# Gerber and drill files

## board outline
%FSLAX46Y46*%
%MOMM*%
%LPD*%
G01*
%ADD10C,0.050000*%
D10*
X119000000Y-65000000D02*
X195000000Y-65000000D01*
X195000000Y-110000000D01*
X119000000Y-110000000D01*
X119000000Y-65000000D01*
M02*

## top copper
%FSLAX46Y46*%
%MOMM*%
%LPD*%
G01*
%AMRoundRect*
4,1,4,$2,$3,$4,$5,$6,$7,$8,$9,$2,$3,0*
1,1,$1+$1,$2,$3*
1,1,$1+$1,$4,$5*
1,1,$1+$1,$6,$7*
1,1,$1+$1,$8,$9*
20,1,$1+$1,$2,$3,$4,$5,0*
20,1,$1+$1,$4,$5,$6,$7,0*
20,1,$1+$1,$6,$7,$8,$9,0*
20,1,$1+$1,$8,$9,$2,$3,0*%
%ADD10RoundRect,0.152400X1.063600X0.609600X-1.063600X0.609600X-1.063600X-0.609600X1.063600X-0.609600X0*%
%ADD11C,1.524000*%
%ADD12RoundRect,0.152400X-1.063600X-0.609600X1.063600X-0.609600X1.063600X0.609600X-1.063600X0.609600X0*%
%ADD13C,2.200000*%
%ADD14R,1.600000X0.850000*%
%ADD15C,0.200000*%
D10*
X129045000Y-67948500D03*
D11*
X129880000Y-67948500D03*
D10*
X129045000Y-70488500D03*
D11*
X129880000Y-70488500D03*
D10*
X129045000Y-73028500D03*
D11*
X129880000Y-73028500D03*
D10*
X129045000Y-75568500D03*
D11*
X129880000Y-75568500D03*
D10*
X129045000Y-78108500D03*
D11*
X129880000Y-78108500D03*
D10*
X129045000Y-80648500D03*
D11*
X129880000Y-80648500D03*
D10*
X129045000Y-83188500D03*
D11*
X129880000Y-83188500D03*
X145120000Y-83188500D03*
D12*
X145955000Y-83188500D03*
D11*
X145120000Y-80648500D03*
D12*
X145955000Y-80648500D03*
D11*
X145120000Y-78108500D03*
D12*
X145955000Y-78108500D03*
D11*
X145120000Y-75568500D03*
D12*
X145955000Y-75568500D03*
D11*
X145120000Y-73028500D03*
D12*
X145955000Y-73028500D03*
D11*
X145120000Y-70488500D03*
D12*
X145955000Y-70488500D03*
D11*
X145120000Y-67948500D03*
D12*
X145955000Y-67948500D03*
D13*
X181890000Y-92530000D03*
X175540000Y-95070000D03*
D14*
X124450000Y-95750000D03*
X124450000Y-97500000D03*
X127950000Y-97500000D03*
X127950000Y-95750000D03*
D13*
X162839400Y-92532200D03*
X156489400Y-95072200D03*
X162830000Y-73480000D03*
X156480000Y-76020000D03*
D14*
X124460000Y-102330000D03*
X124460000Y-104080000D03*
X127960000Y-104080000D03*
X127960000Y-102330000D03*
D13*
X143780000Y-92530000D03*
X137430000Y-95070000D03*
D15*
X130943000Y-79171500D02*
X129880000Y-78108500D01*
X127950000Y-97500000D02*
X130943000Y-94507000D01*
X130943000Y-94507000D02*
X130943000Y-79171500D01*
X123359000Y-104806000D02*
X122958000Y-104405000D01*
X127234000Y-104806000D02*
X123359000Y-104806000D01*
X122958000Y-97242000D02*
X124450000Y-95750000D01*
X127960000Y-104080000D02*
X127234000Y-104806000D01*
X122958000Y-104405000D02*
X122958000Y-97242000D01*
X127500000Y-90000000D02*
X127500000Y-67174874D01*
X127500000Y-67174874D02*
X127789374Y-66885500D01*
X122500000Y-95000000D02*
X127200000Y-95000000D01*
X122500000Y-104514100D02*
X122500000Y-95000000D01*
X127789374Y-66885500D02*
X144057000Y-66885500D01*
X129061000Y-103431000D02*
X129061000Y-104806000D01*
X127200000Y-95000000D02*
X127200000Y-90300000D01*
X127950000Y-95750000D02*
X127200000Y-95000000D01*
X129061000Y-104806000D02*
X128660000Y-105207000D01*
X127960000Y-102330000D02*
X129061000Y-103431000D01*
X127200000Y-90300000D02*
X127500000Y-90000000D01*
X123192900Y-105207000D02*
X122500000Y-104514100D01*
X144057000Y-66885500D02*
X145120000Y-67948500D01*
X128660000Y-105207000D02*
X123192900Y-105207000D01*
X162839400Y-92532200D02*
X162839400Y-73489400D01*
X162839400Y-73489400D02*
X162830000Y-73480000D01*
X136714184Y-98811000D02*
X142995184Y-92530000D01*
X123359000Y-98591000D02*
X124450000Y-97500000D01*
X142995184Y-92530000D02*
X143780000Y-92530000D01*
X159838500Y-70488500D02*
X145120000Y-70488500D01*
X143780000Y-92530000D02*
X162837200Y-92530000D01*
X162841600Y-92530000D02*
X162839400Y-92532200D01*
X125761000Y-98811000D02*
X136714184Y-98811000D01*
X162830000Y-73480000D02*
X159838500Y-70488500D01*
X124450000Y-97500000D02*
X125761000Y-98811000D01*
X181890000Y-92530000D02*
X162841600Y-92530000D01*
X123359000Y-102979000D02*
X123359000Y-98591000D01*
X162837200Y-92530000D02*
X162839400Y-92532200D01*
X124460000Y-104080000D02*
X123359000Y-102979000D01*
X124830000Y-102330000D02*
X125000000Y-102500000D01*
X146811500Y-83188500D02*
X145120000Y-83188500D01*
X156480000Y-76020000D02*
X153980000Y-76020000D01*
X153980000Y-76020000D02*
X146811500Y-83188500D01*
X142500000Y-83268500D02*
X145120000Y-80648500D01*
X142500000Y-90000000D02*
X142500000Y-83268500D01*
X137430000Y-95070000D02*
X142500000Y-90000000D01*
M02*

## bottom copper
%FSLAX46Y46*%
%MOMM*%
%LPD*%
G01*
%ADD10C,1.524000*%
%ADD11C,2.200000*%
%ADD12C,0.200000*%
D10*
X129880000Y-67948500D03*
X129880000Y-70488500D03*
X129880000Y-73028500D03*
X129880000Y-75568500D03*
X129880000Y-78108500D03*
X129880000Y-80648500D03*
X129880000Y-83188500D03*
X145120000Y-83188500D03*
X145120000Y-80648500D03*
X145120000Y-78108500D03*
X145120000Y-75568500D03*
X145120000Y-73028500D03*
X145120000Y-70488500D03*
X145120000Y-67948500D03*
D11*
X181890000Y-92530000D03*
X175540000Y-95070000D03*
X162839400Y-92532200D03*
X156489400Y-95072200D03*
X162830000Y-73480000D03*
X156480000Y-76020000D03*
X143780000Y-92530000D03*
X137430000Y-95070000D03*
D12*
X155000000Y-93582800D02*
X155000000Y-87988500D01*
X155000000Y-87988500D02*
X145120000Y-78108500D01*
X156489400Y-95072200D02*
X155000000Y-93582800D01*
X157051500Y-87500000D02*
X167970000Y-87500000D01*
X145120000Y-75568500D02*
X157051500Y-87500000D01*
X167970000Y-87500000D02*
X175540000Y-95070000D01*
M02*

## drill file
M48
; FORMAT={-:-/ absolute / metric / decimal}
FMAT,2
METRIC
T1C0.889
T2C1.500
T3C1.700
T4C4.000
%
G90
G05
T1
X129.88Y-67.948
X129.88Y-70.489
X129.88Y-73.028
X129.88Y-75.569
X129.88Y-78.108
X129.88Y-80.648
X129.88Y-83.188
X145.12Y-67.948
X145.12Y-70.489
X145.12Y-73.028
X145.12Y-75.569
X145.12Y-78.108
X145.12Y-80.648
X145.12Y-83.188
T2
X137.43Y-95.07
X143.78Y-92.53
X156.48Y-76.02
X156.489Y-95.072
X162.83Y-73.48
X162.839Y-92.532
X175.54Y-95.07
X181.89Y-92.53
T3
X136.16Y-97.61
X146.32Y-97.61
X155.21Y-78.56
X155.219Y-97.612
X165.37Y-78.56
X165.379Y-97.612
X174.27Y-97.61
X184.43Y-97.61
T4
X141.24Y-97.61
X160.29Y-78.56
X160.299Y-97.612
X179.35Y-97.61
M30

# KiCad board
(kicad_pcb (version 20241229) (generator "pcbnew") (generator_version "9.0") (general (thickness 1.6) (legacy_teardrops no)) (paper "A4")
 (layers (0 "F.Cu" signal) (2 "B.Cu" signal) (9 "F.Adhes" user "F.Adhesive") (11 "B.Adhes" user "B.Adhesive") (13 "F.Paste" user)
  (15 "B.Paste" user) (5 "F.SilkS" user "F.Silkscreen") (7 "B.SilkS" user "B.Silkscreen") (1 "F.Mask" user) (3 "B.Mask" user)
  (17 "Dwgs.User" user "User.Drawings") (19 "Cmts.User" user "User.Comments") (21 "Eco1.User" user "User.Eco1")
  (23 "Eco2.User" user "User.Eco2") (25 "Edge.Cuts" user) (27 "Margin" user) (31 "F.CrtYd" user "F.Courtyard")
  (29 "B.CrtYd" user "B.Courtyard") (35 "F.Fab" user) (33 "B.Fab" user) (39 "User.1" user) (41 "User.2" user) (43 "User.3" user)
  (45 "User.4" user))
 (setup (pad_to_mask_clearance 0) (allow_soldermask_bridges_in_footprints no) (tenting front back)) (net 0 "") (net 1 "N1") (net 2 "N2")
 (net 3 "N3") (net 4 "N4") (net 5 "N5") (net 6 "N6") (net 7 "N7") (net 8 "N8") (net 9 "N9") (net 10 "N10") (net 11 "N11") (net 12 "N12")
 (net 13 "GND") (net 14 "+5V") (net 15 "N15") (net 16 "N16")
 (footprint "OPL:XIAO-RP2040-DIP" (layer "F.Cu") (at 137.5 75.5685)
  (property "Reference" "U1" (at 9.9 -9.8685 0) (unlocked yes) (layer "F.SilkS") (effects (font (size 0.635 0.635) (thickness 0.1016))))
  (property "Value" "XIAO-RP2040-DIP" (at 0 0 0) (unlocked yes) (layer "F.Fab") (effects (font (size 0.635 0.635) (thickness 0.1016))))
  (pad "1" smd roundrect (at -8.455 -7.62 180) (size 2.432 1.524) (layers "F.Cu" "F.Mask") (roundrect_rratio 0.1) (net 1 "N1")
   (thermal_bridge_angle 45))
  (pad "1" thru_hole circle (at -7.62 -7.62 180) (size 1.524 1.524) (drill 0.889) (layers "*.Cu" "*.Mask") (remove_unused_layers no)
   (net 1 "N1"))
  (pad "2" smd roundrect (at -8.455 -5.08 180) (size 2.432 1.524) (layers "F.Cu" "F.Mask") (roundrect_rratio 0.1) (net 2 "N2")
   (thermal_bridge_angle 45))
  (pad "2" thru_hole circle (at -7.62 -5.08 180) (size 1.524 1.524) (drill 0.889) (layers "*.Cu" "*.Mask") (remove_unused_layers no)
   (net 2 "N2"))
  (pad "3" smd roundrect (at -8.455 -2.54 180) (size 2.432 1.524) (layers "F.Cu" "F.Mask") (roundrect_rratio 0.1) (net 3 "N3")
   (thermal_bridge_angle 45))
  (pad "3" thru_hole circle (at -7.62 -2.54 180) (size 1.524 1.524) (drill 0.889) (layers "*.Cu" "*.Mask") (remove_unused_layers no)
   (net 3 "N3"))
  (pad "4" smd roundrect (at -8.455 0 180) (size 2.432 1.524) (layers "F.Cu" "F.Mask") (roundrect_rratio 0.1) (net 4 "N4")
   (thermal_bridge_angle 45))
  (pad "4" thru_hole circle (at -7.62 0 180) (size 1.524 1.524) (drill 0.889) (layers "*.Cu" "*.Mask") (remove_unused_layers no)
   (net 4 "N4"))
  (pad "5" smd roundrect (at -8.455 2.54 180) (size 2.432 1.524) (layers "F.Cu" "F.Mask") (roundrect_rratio 0.1) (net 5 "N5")
   (thermal_bridge_angle 45))
  (pad "5" thru_hole circle (at -7.62 2.54 180) (size 1.524 1.524) (drill 0.889) (layers "*.Cu" "*.Mask") (remove_unused_layers no)
   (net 5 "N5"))
  (pad "6" smd roundrect (at -8.455 5.08 180) (size 2.432 1.524) (layers "F.Cu" "F.Mask") (roundrect_rratio 0.1) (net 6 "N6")
   (thermal_bridge_angle 45))
  (pad "6" thru_hole circle (at -7.62 5.08 180) (size 1.524 1.524) (drill 0.889) (layers "*.Cu" "*.Mask") (remove_unused_layers no)
   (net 6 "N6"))
  (pad "7" smd roundrect (at -8.455 7.62 180) (size 2.432 1.524) (layers "F.Cu" "F.Mask") (roundrect_rratio 0.1) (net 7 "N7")
   (thermal_bridge_angle 45))
  (pad "7" thru_hole circle (at -7.62 7.62 180) (size 1.524 1.524) (drill 0.889) (layers "*.Cu" "*.Mask") (remove_unused_layers no)
   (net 7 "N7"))
  (pad "8" thru_hole circle (at 7.62 7.62) (size 1.524 1.524) (drill 0.889) (layers "*.Cu" "*.Mask") (remove_unused_layers no) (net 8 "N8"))
  (pad "8" smd roundrect (at 8.455 7.62) (size 2.432 1.524) (layers "F.Cu" "F.Mask") (roundrect_rratio 0.1) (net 8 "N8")
   (thermal_bridge_angle 45))
  (pad "9" thru_hole circle (at 7.62 5.08) (size 1.524 1.524) (drill 0.889) (layers "*.Cu" "*.Mask") (remove_unused_layers no) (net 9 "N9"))
  (pad "9" smd roundrect (at 8.455 5.08) (size 2.432 1.524) (layers "F.Cu" "F.Mask") (roundrect_rratio 0.1) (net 9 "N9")
   (thermal_bridge_angle 45))
  (pad "10" thru_hole circle (at 7.62 2.54) (size 1.524 1.524) (drill 0.889) (layers "*.Cu" "*.Mask") (remove_unused_layers no)
   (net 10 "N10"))
  (pad "10" smd roundrect (at 8.455 2.54) (size 2.432 1.524) (layers "F.Cu" "F.Mask") (roundrect_rratio 0.1) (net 10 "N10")
   (thermal_bridge_angle 45))
  (pad "11" thru_hole circle (at 7.62 0) (size 1.524 1.524) (drill 0.889) (layers "*.Cu" "*.Mask") (remove_unused_layers no) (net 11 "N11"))
  (pad "11" smd roundrect (at 8.455 0) (size 2.432 1.524) (layers "F.Cu" "F.Mask") (roundrect_rratio 0.1) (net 11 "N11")
   (thermal_bridge_angle 45))
  (pad "12" thru_hole circle (at 7.62 -2.54) (size 1.524 1.524) (drill 0.889) (layers "*.Cu" "*.Mask") (remove_unused_layers no)
   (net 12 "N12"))
  (pad "12" smd roundrect (at 8.455 -2.54) (size 2.432 1.524) (layers "F.Cu" "F.Mask") (roundrect_rratio 0.1) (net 12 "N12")
   (thermal_bridge_angle 45))
  (pad "13" thru_hole circle (at 7.62 -5.08) (size 1.524 1.524) (drill 0.889) (layers "*.Cu" "*.Mask") (remove_unused_layers no)
   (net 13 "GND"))
  (pad "13" smd roundrect (at 8.455 -5.08) (size 2.432 1.524) (layers "F.Cu" "F.Mask") (roundrect_rratio 0.1) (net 13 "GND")
   (thermal_bridge_angle 45))
  (pad "14" thru_hole circle (at 7.62 -7.62) (size 1.524 1.524) (drill 0.889) (layers "*.Cu" "*.Mask") (remove_unused_layers no)
   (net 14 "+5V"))
  (pad "14" smd roundrect (at 8.455 -7.62) (size 2.432 1.524) (layers "F.Cu" "F.Mask") (roundrect_rratio 0.1) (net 14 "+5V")
   (thermal_bridge_angle 45)))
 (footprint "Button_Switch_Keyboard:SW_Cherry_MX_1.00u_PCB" (layer "F.Cu") (at 181.89 92.53)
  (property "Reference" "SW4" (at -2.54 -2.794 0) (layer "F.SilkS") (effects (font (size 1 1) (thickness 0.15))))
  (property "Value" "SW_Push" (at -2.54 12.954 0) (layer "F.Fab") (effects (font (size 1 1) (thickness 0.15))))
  (pad "" np_thru_hole circle (at -7.62 5.08) (size 1.7 1.7) (drill 1.7) (layers "*.Cu" "*.Mask"))
  (pad "" np_thru_hole circle (at -2.54 5.08) (size 4 4) (drill 4) (layers "*.Cu" "*.Mask"))
  (pad "" np_thru_hole circle (at 2.54 5.08) (size 1.7 1.7) (drill 1.7) (layers "*.Cu" "*.Mask"))
  (pad "1" thru_hole circle (at 0 0) (size 2.2 2.2) (drill 1.5) (layers "*.Cu" "*.Mask") (remove_unused_layers no) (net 13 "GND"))
  (pad "2" thru_hole circle (at -6.35 2.54) (size 2.2 2.2) (drill 1.5) (layers "*.Cu" "*.Mask") (remove_unused_layers no) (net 11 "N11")))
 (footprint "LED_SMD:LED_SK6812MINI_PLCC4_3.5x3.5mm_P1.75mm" (layer "F.Cu") (at 126.2 96.625)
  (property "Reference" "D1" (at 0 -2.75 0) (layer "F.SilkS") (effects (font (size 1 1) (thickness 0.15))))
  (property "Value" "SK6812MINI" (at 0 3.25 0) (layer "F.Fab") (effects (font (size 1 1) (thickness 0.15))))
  (pad "1" smd rect (at -1.75 -0.875) (size 1.6 0.85) (layers "F.Cu" "F.Mask" "F.Paste") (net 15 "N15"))
  (pad "2" smd rect (at -1.75 0.875) (size 1.6 0.85) (layers "F.Cu" "F.Mask" "F.Paste") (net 13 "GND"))
  (pad "3" smd rect (at 1.75 0.875) (size 1.6 0.85) (layers "F.Cu" "F.Mask" "F.Paste") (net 5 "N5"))
  (pad "4" smd rect (at 1.75 -0.875) (size 1.6 0.85) (layers "F.Cu" "F.Mask" "F.Paste") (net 14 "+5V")))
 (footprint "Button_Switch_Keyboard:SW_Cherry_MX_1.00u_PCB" (layer "F.Cu") (at 162.8394 92.5322)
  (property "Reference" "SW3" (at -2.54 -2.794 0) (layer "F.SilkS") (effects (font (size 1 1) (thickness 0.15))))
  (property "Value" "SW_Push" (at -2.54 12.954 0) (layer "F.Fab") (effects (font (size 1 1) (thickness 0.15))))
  (pad "" np_thru_hole circle (at -7.62 5.08) (size 1.7 1.7) (drill 1.7) (layers "*.Cu" "*.Mask"))
  (pad "" np_thru_hole circle (at -2.54 5.08) (size 4 4) (drill 4) (layers "*.Cu" "*.Mask"))
  (pad "" np_thru_hole circle (at 2.54 5.08) (size 1.7 1.7) (drill 1.7) (layers "*.Cu" "*.Mask"))
  (pad "1" thru_hole circle (at 0 0) (size 2.2 2.2) (drill 1.5) (layers "*.Cu" "*.Mask") (remove_unused_layers no) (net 13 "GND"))
  (pad "2" thru_hole circle (at -6.35 2.54) (size 2.2 2.2) (drill 1.5) (layers "*.Cu" "*.Mask") (remove_unused_layers no) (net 10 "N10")))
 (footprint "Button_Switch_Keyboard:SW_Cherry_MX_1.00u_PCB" (layer "F.Cu") (at 162.83 73.48)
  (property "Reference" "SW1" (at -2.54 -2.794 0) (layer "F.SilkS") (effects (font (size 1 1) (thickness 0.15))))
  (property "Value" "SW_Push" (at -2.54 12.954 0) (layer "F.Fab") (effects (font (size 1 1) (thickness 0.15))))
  (pad "" np_thru_hole circle (at -7.62 5.08) (size 1.7 1.7) (drill 1.7) (layers "*.Cu" "*.Mask"))
  (pad "" np_thru_hole circle (at -2.54 5.08) (size 4 4) (drill 4) (layers "*.Cu" "*.Mask"))
  (pad "" np_thru_hole circle (at 2.54 5.08) (size 1.7 1.7) (drill 1.7) (layers "*.Cu" "*.Mask"))
  (pad "1" thru_hole circle (at 0 0) (size 2.2 2.2) (drill 1.5) (layers "*.Cu" "*.Mask") (remove_unused_layers no) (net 13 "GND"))
  (pad "2" thru_hole circle (at -6.35 2.54) (size 2.2 2.2) (drill 1.5) (layers "*.Cu" "*.Mask") (remove_unused_layers no) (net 8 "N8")))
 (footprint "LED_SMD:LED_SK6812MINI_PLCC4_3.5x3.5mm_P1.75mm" (layer "F.Cu") (at 126.21 103.205)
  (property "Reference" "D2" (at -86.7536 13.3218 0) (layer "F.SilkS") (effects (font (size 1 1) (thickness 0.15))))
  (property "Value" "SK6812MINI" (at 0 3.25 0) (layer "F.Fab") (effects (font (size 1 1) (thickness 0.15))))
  (pad "1" smd rect (at -1.75 -0.875) (size 1.6 0.85) (layers "F.Cu" "F.Mask" "F.Paste") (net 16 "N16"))
  (pad "2" smd rect (at -1.75 0.875) (size 1.6 0.85) (layers "F.Cu" "F.Mask" "F.Paste") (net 13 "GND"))
  (pad "3" smd rect (at 1.75 0.875) (size 1.6 0.85) (layers "F.Cu" "F.Mask" "F.Paste") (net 15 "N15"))
  (pad "4" smd rect (at 1.75 -0.875) (size 1.6 0.85) (layers "F.Cu" "F.Mask" "F.Paste") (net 14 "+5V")))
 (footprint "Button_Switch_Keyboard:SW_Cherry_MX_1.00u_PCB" (layer "F.Cu") (at 143.78 92.53)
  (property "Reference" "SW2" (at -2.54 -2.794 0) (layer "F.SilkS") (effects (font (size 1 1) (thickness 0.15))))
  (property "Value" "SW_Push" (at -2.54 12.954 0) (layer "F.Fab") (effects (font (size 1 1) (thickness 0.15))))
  (pad "" np_thru_hole circle (at -7.62 5.08) (size 1.7 1.7) (drill 1.7) (layers "*.Cu" "*.Mask"))
  (pad "" np_thru_hole circle (at -2.54 5.08) (size 4 4) (drill 4) (layers "*.Cu" "*.Mask"))
  (pad "" np_thru_hole circle (at 2.54 5.08) (size 1.7 1.7) (drill 1.7) (layers "*.Cu" "*.Mask"))
  (pad "1" thru_hole circle (at 0 0) (size 2.2 2.2) (drill 1.5) (layers "*.Cu" "*.Mask") (remove_unused_layers no) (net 13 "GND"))
  (pad "2" thru_hole circle (at -6.35 2.54) (size 2.2 2.2) (drill 1.5) (layers "*.Cu" "*.Mask") (remove_unused_layers no) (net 9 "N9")))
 (gr_rect (start 119 65) (end 195 110) (stroke (width 0.05) (type default)) (fill no) (layer "Edge.Cuts"))
 (segment (start 130.943 79.1715) (end 129.88 78.1085) (width 0.2) (layer "F.Cu") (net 5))
 (segment (start 127.95 97.5) (end 130.943 94.507) (width 0.2) (layer "F.Cu") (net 5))
 (segment (start 130.943 94.507) (end 130.943 79.1715) (width 0.2) (layer "F.Cu") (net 5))
 (segment (start 123.359 104.806) (end 122.958 104.405) (width 0.2) (layer "F.Cu") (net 15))
 (segment (start 127.234 104.806) (end 123.359 104.806) (width 0.2) (layer "F.Cu") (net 15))
 (segment (start 122.958 97.242) (end 124.45 95.75) (width 0.2) (layer "F.Cu") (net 15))
 (segment (start 127.96 104.08) (end 127.234 104.806) (width 0.2) (layer "F.Cu") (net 15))
 (segment (start 122.958 104.405) (end 122.958 97.242) (width 0.2) (layer "F.Cu") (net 15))
 (segment (start 127.5 90) (end 127.5 67.174874) (width 0.2) (layer "F.Cu") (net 14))
 (segment (start 127.5 67.174874) (end 127.789374 66.8855) (width 0.2) (layer "F.Cu") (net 14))
 (segment (start 122.5 95) (end 127.2 95) (width 0.2) (layer "F.Cu") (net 14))
 (segment (start 122.5 104.5141) (end 122.5 95) (width 0.2) (layer "F.Cu") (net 14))
 (segment (start 127.789374 66.8855) (end 144.057 66.8855) (width 0.2) (layer "F.Cu") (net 14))
 (segment (start 129.061 103.431) (end 129.061 104.806) (width 0.2) (layer "F.Cu") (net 14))
 (segment (start 127.2 95) (end 127.2 90.3) (width 0.2) (layer "F.Cu") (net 14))
 (segment (start 127.95 95.75) (end 127.2 95) (width 0.2) (layer "F.Cu") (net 14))
 (segment (start 129.061 104.806) (end 128.66 105.207) (width 0.2) (layer "F.Cu") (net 14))
 (segment (start 127.96 102.33) (end 129.061 103.431) (width 0.2) (layer "F.Cu") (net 14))
 (segment (start 127.2 90.3) (end 127.5 90) (width 0.2) (layer "F.Cu") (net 14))
 (segment (start 123.1929 105.207) (end 122.5 104.5141) (width 0.2) (layer "F.Cu") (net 14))
 (segment (start 144.057 66.8855) (end 145.12 67.9485) (width 0.2) (layer "F.Cu") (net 14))
 (segment (start 128.66 105.207) (end 123.1929 105.207) (width 0.2) (layer "F.Cu") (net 14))
 (segment (start 162.8394 92.5322) (end 162.8394 73.4894) (width 0.2) (layer "F.Cu") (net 13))
 (segment (start 162.8394 73.4894) (end 162.83 73.48) (width 0.2) (layer "F.Cu") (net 13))
 (segment (start 136.714184 98.811) (end 142.995184 92.53) (width 0.2) (layer "F.Cu") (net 13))
 (segment (start 123.359 98.591) (end 124.45 97.5) (width 0.2) (layer "F.Cu") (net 13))
 (segment (start 142.995184 92.53) (end 143.78 92.53) (width 0.2) (layer "F.Cu") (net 13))
 (segment (start 159.8385 70.4885) (end 145.12 70.4885) (width 0.2) (layer "F.Cu") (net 13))
 (segment (start 143.78 92.53) (end 162.8372 92.53) (width 0.2) (layer "F.Cu") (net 13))
 (segment (start 162.8416 92.53) (end 162.8394 92.5322) (width 0.2) (layer "F.Cu") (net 13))
 (segment (start 125.761 98.811) (end 136.714184 98.811) (width 0.2) (layer "F.Cu") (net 13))
 (segment (start 162.83 73.48) (end 159.8385 70.4885) (width 0.2) (layer "F.Cu") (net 13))
 (segment (start 124.45 97.5) (end 125.761 98.811) (width 0.2) (layer "F.Cu") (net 13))
 (segment (start 181.89 92.53) (end 162.8416 92.53) (width 0.2) (layer "F.Cu") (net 13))
 (segment (start 123.359 102.979) (end 123.359 98.591) (width 0.2) (layer "F.Cu") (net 13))
 (segment (start 162.8372 92.53) (end 162.8394 92.5322) (width 0.2) (layer "F.Cu") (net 13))
 (segment (start 124.46 104.08) (end 123.359 102.979) (width 0.2) (layer "F.Cu") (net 13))
 (segment (start 124.83 102.33) (end 125 102.5) (width 0.2) (layer "F.Cu") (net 16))
 (segment (start 146.8115 83.1885) (end 145.12 83.1885) (width 0.2) (layer "F.Cu") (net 8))
 (segment (start 156.48 76.02) (end 153.98 76.02) (width 0.2) (layer "F.Cu") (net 8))
 (segment (start 153.98 76.02) (end 146.8115 83.1885) (width 0.2) (layer "F.Cu") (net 8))
 (segment (start 142.5 83.2685) (end 145.12 80.6485) (width 0.2) (layer "F.Cu") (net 9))
 (segment (start 142.5 90) (end 142.5 83.2685) (width 0.2) (layer "F.Cu") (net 9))
 (segment (start 137.43 95.07) (end 142.5 90) (width 0.2) (layer "F.Cu") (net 9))
 (segment (start 155 93.5828) (end 155 87.9885) (width 0.2) (layer "B.Cu") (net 10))
 (segment (start 155 87.9885) (end 145.12 78.1085) (width 0.2) (layer "B.Cu") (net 10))
 (segment (start 156.4894 95.0722) (end 155 93.5828) (width 0.2) (layer "B.Cu") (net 10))
 (segment (start 157.0515 87.5) (end 167.97 87.5) (width 0.2) (layer "B.Cu") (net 11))
 (segment (start 145.12 75.5685) (end 157.0515 87.5) (width 0.2) (layer "B.Cu") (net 11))
 (segment (start 167.97 87.5) (end 175.54 95.07) (width 0.2) (layer "B.Cu") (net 11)))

